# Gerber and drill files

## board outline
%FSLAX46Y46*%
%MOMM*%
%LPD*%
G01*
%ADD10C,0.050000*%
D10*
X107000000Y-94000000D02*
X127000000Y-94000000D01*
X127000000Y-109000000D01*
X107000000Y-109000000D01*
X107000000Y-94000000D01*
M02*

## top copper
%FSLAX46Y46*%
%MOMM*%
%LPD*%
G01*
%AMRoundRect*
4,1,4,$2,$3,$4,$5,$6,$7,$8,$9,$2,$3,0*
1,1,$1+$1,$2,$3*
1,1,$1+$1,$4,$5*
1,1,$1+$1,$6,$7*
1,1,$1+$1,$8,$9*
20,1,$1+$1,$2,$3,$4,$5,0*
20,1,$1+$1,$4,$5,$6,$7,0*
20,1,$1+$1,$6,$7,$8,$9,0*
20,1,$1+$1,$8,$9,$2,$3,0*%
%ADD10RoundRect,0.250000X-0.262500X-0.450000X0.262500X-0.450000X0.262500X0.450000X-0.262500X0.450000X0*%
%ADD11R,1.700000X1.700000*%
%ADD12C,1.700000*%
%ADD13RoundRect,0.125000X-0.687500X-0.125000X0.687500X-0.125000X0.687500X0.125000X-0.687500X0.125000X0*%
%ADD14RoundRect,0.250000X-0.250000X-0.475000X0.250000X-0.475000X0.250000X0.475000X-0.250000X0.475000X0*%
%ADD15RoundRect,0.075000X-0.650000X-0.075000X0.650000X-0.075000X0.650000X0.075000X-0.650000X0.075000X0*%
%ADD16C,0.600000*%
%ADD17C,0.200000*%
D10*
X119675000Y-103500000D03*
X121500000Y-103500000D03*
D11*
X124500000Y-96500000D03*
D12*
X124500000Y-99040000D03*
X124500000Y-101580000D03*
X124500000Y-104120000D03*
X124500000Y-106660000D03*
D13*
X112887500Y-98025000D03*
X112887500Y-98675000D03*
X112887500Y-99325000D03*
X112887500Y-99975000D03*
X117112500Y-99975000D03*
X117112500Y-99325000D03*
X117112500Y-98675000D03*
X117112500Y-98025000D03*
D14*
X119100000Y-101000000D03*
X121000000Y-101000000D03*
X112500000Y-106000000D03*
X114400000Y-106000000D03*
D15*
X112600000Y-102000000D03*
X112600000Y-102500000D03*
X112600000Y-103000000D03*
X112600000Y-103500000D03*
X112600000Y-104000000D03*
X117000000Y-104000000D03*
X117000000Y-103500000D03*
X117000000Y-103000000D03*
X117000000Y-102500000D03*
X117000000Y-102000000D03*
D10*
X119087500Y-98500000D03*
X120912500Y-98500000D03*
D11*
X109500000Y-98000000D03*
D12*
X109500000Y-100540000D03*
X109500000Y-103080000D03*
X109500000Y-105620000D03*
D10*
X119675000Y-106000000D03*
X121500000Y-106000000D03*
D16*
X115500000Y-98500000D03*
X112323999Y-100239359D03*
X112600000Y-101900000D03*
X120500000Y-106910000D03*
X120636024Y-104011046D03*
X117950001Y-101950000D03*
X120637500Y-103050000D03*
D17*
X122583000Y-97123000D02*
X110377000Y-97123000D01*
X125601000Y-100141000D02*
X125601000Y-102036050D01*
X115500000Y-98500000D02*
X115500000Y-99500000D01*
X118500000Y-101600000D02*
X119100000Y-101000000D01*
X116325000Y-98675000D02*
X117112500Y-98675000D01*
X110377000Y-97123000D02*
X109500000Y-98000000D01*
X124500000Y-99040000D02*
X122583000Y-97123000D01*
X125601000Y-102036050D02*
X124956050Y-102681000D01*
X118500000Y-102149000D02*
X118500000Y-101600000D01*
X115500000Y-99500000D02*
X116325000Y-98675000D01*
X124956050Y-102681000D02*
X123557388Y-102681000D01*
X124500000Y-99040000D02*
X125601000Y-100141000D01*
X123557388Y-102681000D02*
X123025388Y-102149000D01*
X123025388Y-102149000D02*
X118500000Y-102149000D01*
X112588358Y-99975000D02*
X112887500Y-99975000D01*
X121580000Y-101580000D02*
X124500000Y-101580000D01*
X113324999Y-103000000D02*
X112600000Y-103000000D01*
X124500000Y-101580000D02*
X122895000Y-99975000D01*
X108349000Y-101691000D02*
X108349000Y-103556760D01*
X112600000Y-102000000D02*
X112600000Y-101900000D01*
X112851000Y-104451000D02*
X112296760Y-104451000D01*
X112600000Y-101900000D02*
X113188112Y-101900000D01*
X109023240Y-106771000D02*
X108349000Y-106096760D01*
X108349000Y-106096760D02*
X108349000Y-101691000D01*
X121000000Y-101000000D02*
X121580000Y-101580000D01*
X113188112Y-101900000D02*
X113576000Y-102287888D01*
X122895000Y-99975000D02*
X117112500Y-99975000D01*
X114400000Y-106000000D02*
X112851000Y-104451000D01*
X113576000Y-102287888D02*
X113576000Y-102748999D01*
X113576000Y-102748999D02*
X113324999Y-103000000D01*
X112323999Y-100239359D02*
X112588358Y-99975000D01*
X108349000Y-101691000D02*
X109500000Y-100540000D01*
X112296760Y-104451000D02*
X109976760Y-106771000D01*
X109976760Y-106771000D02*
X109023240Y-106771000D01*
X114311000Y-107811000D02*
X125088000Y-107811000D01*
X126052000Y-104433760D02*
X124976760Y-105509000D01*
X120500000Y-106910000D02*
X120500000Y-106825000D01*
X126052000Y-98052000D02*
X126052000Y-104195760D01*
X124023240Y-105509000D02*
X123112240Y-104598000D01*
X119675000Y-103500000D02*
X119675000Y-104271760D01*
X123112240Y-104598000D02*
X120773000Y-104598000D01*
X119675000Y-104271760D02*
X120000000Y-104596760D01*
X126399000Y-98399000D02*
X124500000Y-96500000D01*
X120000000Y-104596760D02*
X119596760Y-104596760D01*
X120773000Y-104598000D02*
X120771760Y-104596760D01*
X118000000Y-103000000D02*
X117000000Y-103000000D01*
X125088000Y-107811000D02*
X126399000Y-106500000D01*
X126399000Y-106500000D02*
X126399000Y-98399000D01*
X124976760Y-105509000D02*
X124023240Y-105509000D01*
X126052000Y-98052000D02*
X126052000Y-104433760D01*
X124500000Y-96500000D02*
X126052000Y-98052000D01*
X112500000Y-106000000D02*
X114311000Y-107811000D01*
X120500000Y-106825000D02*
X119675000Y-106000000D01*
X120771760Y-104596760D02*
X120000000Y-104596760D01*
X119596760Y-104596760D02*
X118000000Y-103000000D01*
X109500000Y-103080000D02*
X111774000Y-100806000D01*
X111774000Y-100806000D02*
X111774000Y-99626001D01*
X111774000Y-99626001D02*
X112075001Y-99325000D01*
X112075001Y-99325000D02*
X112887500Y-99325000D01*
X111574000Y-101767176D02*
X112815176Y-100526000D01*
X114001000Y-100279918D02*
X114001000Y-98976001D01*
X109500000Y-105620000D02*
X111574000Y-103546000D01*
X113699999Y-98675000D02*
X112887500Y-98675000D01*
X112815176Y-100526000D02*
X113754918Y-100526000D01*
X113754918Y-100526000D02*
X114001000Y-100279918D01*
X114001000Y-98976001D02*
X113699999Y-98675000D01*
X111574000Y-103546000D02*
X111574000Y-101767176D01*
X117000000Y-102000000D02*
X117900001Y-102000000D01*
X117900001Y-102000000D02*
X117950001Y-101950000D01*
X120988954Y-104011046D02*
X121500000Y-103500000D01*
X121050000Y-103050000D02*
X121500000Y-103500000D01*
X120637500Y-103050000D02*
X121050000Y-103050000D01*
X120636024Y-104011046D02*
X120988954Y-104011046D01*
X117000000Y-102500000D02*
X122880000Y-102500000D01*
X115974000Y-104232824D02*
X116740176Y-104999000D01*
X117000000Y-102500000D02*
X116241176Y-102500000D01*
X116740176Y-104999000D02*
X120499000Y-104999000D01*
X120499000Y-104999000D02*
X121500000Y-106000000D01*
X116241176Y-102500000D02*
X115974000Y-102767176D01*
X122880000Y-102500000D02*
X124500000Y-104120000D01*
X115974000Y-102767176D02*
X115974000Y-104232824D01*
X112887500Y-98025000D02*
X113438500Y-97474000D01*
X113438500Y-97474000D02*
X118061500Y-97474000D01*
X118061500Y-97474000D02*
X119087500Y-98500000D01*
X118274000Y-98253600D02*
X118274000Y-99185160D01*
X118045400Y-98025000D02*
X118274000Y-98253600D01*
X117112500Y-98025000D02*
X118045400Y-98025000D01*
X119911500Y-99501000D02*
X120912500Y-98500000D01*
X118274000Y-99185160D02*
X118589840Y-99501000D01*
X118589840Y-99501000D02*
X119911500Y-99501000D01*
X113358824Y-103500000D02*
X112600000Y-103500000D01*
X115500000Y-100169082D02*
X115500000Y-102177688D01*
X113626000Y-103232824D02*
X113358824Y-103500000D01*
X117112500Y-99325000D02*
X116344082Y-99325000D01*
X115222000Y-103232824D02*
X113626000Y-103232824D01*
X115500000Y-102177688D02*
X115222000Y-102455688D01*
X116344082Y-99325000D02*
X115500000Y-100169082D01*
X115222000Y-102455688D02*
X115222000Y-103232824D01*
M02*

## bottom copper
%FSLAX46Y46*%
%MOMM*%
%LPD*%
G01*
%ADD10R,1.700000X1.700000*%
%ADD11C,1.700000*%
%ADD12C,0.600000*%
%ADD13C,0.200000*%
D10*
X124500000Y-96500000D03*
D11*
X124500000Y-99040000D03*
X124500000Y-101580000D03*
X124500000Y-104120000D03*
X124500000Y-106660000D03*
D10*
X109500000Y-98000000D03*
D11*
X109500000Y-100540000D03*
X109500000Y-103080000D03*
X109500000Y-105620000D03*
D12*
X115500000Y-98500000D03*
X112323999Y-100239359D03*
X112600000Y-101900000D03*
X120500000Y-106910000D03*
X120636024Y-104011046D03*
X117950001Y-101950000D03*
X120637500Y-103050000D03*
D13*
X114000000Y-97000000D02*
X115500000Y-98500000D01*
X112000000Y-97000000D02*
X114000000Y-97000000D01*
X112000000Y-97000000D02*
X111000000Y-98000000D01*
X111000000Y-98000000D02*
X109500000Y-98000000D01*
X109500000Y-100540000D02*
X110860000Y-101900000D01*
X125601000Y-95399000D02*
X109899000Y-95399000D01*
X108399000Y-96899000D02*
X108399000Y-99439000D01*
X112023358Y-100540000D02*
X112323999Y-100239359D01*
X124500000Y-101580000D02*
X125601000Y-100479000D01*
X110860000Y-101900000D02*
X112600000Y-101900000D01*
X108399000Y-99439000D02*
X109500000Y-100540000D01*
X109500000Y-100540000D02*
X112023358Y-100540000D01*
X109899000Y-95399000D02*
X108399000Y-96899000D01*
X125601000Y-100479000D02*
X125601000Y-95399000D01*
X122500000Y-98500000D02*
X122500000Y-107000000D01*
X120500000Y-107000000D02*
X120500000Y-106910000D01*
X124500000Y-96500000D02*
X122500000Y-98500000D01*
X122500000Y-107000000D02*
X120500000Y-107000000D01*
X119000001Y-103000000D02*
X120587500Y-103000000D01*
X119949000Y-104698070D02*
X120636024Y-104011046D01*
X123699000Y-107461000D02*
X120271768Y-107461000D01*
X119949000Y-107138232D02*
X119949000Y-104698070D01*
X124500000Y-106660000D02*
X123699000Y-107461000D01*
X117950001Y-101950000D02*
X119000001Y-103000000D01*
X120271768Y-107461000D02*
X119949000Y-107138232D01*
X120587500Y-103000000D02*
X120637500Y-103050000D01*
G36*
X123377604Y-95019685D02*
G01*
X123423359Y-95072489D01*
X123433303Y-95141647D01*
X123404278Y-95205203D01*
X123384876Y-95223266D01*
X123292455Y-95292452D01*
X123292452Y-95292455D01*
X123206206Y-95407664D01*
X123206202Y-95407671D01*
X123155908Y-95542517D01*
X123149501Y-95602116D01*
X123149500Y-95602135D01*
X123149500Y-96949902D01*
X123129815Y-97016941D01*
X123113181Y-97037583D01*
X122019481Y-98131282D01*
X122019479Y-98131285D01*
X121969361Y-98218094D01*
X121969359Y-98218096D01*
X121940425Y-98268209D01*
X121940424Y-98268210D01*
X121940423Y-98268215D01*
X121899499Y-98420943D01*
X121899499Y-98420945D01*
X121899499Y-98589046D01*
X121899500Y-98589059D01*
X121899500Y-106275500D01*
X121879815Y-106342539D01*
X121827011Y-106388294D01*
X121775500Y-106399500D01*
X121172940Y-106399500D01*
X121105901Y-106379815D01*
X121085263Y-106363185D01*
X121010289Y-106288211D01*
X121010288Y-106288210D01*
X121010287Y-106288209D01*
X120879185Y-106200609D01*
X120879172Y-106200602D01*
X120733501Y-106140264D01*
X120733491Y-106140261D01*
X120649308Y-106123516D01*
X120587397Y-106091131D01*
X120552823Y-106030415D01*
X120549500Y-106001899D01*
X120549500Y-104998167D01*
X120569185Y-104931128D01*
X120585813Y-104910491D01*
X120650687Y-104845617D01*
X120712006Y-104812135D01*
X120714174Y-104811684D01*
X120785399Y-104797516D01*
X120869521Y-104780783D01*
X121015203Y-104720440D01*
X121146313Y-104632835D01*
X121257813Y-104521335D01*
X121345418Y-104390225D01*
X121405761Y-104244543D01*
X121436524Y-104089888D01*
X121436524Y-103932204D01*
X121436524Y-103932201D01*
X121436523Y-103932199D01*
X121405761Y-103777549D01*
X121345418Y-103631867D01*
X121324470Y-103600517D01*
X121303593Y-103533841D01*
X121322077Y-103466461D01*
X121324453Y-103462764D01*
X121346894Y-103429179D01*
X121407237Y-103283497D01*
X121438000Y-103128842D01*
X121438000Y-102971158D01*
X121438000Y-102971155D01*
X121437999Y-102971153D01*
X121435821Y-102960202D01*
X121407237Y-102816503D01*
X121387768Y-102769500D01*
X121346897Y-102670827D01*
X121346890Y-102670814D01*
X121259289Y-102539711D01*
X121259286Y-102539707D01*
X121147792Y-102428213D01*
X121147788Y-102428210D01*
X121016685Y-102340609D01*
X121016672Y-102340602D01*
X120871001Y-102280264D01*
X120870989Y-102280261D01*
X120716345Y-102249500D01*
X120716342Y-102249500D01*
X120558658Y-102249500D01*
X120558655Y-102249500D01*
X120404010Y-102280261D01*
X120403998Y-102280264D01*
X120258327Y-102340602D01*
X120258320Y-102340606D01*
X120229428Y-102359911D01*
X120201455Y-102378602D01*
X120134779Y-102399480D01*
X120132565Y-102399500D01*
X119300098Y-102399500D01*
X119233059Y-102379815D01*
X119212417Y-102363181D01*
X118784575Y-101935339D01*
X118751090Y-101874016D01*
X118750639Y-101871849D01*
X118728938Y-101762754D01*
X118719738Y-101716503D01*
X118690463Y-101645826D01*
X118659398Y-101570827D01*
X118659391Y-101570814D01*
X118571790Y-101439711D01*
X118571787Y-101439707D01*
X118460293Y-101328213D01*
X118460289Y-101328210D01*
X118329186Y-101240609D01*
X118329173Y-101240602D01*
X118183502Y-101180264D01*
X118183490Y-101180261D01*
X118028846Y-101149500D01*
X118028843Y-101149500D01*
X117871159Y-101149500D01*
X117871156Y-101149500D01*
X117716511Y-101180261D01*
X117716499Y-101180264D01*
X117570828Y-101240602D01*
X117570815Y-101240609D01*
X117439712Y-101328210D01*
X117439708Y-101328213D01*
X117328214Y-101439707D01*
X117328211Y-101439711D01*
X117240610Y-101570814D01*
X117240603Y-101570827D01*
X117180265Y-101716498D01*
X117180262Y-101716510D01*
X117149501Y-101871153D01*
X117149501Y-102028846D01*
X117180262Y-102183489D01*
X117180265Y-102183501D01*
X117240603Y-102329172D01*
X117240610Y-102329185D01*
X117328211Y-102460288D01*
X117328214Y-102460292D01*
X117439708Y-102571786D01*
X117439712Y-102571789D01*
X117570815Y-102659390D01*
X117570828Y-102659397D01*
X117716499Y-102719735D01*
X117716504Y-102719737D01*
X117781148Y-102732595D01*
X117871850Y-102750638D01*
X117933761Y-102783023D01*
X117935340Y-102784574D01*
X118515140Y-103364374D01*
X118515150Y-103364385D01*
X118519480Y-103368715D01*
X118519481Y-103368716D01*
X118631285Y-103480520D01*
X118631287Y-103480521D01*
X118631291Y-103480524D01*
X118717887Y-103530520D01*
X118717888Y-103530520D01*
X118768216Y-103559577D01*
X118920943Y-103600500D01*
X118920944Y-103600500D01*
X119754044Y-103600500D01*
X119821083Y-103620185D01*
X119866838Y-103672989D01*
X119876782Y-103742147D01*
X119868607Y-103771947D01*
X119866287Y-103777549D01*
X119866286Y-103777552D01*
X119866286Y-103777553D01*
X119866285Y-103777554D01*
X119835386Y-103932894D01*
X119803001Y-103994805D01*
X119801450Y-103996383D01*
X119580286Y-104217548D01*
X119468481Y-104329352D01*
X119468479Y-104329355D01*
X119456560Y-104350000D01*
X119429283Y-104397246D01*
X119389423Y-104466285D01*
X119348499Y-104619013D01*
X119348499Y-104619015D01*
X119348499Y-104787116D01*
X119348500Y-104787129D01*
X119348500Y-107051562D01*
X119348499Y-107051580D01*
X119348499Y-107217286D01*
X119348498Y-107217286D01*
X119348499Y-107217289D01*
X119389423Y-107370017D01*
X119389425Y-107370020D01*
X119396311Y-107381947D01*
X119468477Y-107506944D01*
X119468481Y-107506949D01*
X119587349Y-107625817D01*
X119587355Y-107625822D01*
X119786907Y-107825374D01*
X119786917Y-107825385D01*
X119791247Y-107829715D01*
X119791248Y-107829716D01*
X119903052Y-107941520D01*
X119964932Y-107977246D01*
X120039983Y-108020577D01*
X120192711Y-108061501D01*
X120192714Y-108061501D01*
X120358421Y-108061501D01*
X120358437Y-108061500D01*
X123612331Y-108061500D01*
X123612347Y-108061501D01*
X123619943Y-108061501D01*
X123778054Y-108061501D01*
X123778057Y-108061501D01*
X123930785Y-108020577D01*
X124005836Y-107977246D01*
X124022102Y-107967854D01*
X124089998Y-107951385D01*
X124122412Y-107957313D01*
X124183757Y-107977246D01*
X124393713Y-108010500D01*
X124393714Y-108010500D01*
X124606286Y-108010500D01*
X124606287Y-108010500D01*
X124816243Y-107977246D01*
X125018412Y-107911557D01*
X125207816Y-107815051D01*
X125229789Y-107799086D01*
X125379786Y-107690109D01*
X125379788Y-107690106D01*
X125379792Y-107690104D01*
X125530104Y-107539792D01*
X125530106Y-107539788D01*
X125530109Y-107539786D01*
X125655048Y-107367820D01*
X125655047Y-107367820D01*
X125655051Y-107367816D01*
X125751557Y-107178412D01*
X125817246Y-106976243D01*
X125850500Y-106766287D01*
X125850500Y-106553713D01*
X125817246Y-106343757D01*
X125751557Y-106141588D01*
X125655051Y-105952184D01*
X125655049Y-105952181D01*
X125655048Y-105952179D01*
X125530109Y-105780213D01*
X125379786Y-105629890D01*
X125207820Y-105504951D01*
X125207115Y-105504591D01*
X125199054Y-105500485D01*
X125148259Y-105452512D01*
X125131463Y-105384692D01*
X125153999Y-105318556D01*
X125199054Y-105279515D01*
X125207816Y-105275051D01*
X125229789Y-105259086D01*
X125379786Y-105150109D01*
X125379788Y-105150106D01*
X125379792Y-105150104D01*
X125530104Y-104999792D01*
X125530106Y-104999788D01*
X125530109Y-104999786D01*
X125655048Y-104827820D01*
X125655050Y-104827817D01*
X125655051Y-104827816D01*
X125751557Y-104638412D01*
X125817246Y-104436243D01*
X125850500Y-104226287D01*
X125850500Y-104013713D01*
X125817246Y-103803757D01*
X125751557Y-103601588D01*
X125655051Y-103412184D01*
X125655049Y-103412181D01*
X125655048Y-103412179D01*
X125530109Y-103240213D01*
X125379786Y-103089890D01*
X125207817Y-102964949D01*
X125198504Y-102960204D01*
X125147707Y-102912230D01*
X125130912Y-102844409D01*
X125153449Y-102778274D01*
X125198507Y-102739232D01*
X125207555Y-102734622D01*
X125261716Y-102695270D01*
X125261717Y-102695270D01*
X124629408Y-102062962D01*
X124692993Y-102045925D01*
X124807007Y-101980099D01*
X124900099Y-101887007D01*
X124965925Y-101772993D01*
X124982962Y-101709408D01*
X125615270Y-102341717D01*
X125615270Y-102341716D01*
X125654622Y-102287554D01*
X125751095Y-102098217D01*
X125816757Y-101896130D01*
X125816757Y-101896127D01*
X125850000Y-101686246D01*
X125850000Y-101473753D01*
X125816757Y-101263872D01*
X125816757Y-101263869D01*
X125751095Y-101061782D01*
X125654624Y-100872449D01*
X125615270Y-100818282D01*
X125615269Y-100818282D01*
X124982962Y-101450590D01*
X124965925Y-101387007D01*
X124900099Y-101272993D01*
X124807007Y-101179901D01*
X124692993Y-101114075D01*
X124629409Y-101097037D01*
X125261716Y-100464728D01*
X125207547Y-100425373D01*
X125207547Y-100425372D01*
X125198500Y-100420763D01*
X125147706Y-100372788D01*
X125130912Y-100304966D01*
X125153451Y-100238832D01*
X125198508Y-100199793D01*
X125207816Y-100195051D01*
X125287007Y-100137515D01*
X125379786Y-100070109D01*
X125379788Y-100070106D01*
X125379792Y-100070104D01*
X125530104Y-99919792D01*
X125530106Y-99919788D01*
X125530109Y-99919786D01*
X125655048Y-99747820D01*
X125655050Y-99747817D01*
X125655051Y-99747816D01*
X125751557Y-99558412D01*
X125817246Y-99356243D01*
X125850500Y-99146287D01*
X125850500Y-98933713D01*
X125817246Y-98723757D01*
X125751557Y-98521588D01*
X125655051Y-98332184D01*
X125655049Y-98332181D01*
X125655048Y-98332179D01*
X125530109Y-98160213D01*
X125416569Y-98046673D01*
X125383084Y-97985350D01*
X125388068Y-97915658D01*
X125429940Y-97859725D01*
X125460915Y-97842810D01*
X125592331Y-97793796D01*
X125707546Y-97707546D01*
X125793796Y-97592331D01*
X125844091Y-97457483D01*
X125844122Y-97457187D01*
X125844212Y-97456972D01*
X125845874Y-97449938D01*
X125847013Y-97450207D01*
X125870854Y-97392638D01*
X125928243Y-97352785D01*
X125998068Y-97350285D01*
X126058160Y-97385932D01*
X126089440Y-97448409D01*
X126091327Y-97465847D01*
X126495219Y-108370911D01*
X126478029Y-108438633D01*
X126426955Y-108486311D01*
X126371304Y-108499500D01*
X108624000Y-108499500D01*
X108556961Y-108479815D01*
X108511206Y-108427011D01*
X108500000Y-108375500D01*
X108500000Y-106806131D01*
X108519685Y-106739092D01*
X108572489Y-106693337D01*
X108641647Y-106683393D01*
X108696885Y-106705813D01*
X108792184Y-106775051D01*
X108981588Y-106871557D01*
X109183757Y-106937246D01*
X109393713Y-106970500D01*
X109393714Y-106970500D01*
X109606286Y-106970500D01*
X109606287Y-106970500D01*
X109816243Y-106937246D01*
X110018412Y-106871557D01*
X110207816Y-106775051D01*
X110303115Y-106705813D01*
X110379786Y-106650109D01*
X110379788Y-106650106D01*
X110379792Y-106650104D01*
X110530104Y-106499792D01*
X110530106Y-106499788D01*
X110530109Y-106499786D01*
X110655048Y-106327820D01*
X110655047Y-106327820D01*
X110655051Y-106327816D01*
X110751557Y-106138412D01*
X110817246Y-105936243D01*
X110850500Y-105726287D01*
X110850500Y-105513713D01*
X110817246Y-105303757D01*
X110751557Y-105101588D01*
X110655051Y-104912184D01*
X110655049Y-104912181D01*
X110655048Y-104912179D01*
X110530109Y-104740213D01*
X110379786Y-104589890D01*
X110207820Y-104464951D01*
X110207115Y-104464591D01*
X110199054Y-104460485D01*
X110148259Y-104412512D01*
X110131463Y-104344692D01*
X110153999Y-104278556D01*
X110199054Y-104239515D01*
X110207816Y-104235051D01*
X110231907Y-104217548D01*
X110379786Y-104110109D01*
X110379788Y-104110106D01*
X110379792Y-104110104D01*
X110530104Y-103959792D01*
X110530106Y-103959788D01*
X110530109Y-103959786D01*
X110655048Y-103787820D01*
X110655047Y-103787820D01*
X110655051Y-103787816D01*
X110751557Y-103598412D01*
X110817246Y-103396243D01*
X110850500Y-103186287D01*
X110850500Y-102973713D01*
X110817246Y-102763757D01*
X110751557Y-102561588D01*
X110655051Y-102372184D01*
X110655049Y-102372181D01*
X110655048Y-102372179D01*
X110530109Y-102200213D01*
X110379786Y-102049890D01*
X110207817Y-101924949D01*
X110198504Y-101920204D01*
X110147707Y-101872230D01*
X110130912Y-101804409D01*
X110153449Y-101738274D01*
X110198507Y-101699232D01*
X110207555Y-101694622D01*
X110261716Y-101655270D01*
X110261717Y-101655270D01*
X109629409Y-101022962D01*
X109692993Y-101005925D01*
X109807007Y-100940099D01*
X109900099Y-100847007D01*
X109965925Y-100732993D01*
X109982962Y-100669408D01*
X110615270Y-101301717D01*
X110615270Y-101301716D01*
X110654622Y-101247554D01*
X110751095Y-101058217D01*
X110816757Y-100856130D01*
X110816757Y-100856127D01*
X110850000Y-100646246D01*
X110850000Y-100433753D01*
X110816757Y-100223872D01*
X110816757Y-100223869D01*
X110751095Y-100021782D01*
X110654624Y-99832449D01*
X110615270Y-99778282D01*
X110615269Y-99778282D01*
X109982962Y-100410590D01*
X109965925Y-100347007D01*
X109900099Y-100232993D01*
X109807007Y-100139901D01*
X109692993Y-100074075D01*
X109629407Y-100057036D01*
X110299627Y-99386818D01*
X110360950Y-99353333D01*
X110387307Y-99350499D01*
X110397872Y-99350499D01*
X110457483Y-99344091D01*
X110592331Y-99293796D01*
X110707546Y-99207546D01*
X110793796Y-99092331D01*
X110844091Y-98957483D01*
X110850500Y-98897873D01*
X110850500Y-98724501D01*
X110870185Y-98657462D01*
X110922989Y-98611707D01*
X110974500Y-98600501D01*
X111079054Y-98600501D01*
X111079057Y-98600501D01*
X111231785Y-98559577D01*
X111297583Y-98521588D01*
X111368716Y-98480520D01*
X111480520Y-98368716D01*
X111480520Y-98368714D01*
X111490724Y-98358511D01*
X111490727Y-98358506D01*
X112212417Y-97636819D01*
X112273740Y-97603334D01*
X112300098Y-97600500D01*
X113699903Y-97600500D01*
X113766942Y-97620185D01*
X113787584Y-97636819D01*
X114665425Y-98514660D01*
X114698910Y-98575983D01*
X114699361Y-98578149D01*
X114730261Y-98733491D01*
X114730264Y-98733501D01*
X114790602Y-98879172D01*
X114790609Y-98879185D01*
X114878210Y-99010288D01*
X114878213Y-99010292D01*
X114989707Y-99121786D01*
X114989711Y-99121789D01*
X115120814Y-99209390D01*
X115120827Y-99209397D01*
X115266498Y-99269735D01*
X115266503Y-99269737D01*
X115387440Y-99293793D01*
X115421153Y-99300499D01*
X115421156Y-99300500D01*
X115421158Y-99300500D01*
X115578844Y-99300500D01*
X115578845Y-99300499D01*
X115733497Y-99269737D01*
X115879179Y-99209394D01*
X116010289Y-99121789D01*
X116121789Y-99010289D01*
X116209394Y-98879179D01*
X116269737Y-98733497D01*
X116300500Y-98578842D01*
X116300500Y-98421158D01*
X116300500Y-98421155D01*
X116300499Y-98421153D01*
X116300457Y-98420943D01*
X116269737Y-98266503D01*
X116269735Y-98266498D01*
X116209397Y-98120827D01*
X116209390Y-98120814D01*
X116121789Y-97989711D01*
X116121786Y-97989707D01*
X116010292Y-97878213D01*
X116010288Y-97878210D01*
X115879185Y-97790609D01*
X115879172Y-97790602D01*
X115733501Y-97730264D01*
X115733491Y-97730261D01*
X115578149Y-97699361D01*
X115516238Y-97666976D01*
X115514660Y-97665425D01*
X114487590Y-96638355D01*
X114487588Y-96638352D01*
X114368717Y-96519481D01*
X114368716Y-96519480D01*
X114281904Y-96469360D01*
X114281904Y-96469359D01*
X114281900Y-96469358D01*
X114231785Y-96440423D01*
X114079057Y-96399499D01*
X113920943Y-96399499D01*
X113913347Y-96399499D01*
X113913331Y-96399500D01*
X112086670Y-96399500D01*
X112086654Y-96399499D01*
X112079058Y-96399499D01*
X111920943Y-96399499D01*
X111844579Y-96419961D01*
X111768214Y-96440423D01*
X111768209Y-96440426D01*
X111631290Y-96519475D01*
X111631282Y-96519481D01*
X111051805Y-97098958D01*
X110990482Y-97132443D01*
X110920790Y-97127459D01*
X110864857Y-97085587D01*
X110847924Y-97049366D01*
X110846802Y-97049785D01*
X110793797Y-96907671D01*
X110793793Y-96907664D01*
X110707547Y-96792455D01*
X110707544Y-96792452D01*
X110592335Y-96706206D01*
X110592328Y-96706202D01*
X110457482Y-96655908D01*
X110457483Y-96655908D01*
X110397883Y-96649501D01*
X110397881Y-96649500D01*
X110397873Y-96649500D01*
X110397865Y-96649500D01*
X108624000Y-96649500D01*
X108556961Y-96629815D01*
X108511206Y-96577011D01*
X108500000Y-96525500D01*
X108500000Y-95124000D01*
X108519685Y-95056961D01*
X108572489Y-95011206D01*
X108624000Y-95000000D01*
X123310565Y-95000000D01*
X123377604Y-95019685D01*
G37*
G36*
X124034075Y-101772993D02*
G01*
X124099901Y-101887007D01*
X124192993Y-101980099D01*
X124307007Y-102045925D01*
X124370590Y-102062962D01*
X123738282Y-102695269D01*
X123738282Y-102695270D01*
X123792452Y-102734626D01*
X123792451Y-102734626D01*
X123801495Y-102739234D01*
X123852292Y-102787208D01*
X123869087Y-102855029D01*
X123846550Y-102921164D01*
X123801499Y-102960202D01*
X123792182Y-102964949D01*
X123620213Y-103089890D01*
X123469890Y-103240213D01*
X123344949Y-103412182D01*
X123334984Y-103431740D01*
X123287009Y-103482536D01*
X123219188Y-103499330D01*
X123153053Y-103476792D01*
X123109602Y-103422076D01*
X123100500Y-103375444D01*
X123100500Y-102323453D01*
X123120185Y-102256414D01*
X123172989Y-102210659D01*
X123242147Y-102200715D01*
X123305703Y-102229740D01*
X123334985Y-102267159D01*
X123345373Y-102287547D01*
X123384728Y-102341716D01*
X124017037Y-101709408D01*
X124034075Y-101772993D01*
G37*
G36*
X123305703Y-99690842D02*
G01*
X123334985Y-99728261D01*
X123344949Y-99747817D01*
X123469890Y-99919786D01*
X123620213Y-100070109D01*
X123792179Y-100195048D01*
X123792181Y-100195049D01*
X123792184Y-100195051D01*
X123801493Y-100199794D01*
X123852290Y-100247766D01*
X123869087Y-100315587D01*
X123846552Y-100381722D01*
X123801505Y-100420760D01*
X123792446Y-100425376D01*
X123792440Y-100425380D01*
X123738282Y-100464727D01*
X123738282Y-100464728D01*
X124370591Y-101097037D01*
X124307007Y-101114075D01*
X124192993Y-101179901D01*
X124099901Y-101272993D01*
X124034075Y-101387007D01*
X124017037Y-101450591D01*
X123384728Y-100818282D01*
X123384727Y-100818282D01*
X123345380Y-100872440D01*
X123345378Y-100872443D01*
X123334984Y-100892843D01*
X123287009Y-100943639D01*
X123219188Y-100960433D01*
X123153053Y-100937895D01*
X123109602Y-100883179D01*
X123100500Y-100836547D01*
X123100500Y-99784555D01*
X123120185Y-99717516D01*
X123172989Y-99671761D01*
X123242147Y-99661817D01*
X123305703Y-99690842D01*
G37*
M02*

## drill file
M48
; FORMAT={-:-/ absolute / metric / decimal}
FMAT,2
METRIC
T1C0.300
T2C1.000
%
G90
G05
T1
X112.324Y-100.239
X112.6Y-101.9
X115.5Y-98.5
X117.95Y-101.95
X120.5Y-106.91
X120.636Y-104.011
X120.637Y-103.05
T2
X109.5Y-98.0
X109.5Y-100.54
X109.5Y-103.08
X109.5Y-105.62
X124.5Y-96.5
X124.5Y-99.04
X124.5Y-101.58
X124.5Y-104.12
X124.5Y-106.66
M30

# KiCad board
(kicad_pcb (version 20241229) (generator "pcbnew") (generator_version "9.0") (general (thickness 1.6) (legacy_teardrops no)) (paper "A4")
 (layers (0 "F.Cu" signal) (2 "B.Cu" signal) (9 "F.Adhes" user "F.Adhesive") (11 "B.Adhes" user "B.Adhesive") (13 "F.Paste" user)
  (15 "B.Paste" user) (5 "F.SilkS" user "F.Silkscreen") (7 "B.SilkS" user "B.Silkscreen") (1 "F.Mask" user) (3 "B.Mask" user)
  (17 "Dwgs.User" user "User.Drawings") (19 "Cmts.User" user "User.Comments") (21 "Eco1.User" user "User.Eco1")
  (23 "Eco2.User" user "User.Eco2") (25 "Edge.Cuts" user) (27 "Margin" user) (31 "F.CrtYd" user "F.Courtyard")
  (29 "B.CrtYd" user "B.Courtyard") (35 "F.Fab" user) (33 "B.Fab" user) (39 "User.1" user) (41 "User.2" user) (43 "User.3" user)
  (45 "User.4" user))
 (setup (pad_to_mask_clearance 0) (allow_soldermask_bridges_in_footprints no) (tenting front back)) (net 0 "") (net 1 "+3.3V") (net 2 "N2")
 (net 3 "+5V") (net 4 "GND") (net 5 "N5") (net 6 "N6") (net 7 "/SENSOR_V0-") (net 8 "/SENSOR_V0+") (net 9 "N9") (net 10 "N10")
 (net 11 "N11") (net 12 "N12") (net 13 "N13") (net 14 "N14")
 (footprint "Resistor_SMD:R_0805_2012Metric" (layer "F.Cu") (at 120.5875 103.5)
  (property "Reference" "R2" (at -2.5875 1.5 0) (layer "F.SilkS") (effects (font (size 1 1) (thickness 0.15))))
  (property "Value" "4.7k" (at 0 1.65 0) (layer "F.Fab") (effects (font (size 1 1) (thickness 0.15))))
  (pad "1" smd roundrect (at -0.9125 0) (size 1.025 1.4) (layers "F.Cu" "F.Mask" "F.Paste") (roundrect_rratio 0.243902) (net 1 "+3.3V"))
  (pad "2" smd roundrect (at 0.9125 0) (size 1.025 1.4) (layers "F.Cu" "F.Mask" "F.Paste") (roundrect_rratio 0.243902) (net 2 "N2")))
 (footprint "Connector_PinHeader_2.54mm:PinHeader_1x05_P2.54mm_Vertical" (layer "F.Cu") (at 124.5 96.5)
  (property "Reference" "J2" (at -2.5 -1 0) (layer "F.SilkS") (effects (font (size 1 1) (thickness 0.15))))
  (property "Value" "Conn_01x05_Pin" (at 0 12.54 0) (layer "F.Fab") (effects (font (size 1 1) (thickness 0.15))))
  (pad "1" thru_hole rect (at 0 0) (size 1.7 1.7) (drill 1) (layers "*.Cu" "*.Mask") (remove_unused_layers no) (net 1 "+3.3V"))
  (pad "2" thru_hole circle (at 0 2.54) (size 1.7 1.7) (drill 1) (layers "*.Cu" "*.Mask") (remove_unused_layers no) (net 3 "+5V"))
  (pad "3" thru_hole circle (at 0 5.08) (size 1.7 1.7) (drill 1) (layers "*.Cu" "*.Mask") (remove_unused_layers no) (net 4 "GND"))
  (pad "4" thru_hole circle (at 0 7.62) (size 1.7 1.7) (drill 1) (layers "*.Cu" "*.Mask") (remove_unused_layers no) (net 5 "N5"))
  (pad "5" thru_hole circle (at 0 10.16) (size 1.7 1.7) (drill 1) (layers "*.Cu" "*.Mask") (remove_unused_layers no) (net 2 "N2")))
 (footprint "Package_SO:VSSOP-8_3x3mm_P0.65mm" (layer "F.Cu") (at 115 99)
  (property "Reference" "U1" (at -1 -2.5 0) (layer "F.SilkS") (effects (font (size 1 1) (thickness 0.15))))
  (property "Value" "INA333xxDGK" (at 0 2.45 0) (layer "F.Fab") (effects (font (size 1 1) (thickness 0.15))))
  (pad "1" smd roundrect (at -2.1125 -0.975) (size 1.625 0.5) (layers "F.Cu" "F.Mask" "F.Paste") (roundrect_rratio 0.25) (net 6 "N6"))
  (pad "2" smd roundrect (at -2.1125 -0.325) (size 1.625 0.5) (layers "F.Cu" "F.Mask" "F.Paste") (roundrect_rratio 0.25)
   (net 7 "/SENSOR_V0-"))
  (pad "3" smd roundrect (at -2.1125 0.325) (size 1.625 0.5) (layers "F.Cu" "F.Mask" "F.Paste") (roundrect_rratio 0.25)
   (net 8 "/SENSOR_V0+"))
  (pad "4" smd roundrect (at -2.1125 0.975) (size 1.625 0.5) (layers "F.Cu" "F.Mask" "F.Paste") (roundrect_rratio 0.25) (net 4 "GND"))
  (pad "5" smd roundrect (at 2.1125 0.975) (size 1.625 0.5) (layers "F.Cu" "F.Mask" "F.Paste") (roundrect_rratio 0.25) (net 4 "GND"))
  (pad "6" smd roundrect (at 2.1125 0.325) (size 1.625 0.5) (layers "F.Cu" "F.Mask" "F.Paste") (roundrect_rratio 0.25) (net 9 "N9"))
  (pad "7" smd roundrect (at 2.1125 -0.325) (size 1.625 0.5) (layers "F.Cu" "F.Mask" "F.Paste") (roundrect_rratio 0.25) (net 3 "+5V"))
  (pad "8" smd roundrect (at 2.1125 -0.975) (size 1.625 0.5) (layers "F.Cu" "F.Mask" "F.Paste") (roundrect_rratio 0.25) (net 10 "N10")))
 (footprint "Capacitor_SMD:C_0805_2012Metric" (layer "F.Cu") (at 120.05 101)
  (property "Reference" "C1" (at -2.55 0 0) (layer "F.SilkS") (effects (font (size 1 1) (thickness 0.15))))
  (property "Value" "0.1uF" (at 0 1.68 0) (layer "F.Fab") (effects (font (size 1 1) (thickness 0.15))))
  (pad "1" smd roundrect (at -0.95 0) (size 1 1.45) (layers "F.Cu" "F.Mask" "F.Paste") (roundrect_rratio 0.25) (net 3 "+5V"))
  (pad "2" smd roundrect (at 0.95 0) (size 1 1.45) (layers "F.Cu" "F.Mask" "F.Paste") (roundrect_rratio 0.25) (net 4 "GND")))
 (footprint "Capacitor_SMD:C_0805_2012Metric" (layer "F.Cu") (at 113.45 106)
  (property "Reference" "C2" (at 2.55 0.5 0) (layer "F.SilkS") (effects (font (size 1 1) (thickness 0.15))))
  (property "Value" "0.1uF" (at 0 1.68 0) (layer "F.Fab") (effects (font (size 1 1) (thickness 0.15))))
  (pad "1" smd roundrect (at -0.95 0) (size 1 1.45) (layers "F.Cu" "F.Mask" "F.Paste") (roundrect_rratio 0.25) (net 1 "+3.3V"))
  (pad "2" smd roundrect (at 0.95 0) (size 1 1.45) (layers "F.Cu" "F.Mask" "F.Paste") (roundrect_rratio 0.25) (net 4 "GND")))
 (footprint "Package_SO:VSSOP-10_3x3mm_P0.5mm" (layer "F.Cu") (at 114.8 103)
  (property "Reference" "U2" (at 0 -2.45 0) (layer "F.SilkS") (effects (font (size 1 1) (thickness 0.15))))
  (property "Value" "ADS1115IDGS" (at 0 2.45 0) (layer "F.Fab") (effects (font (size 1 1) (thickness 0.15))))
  (pad "1" smd roundrect (at -2.2 -1) (size 1.45 0.3) (layers "F.Cu" "F.Mask" "F.Paste") (roundrect_rratio 0.25) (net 4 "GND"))
  (pad "2" smd roundrect (at -2.2 -0.5) (size 1.45 0.3) (layers "F.Cu" "F.Mask" "F.Paste") (roundrect_rratio 0.25) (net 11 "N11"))
  (pad "3" smd roundrect (at -2.2 0) (size 1.45 0.3) (layers "F.Cu" "F.Mask" "F.Paste") (roundrect_rratio 0.25) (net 4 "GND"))
  (pad "4" smd roundrect (at -2.2 0.5) (size 1.45 0.3) (layers "F.Cu" "F.Mask" "F.Paste") (roundrect_rratio 0.25) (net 9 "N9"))
  (pad "5" smd roundrect (at -2.2 1) (size 1.45 0.3) (layers "F.Cu" "F.Mask" "F.Paste") (roundrect_rratio 0.25) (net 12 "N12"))
  (pad "6" smd roundrect (at 2.2 1) (size 1.45 0.3) (layers "F.Cu" "F.Mask" "F.Paste") (roundrect_rratio 0.25) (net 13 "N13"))
  (pad "7" smd roundrect (at 2.2 0.5) (size 1.45 0.3) (layers "F.Cu" "F.Mask" "F.Paste") (roundrect_rratio 0.25) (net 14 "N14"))
  (pad "8" smd roundrect (at 2.2 0) (size 1.45 0.3) (layers "F.Cu" "F.Mask" "F.Paste") (roundrect_rratio 0.25) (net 1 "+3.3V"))
  (pad "9" smd roundrect (at 2.2 -0.5) (size 1.45 0.3) (layers "F.Cu" "F.Mask" "F.Paste") (roundrect_rratio 0.25) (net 5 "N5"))
  (pad "10" smd roundrect (at 2.2 -1) (size 1.45 0.3) (layers "F.Cu" "F.Mask" "F.Paste") (roundrect_rratio 0.25) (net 2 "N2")))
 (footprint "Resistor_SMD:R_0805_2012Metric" (layer "F.Cu") (at 120 98.5)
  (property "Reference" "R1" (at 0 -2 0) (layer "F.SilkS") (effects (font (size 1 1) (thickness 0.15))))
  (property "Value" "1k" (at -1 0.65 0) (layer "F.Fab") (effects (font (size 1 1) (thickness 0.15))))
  (pad "1" smd roundrect (at -0.9125 0) (size 1.025 1.4) (layers "F.Cu" "F.Mask" "F.Paste") (roundrect_rratio 0.243902) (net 6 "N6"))
  (pad "2" smd roundrect (at 0.9125 0) (size 1.025 1.4) (layers "F.Cu" "F.Mask" "F.Paste") (roundrect_rratio 0.243902) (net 10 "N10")))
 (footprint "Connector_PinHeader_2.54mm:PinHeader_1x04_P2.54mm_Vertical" (layer "F.Cu") (at 109.5 98)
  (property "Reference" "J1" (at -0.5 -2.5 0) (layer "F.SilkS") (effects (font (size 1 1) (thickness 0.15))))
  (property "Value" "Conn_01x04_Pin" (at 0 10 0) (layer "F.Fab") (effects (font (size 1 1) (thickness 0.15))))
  (pad "1" thru_hole rect (at 0 0) (size 1.7 1.7) (drill 1) (layers "*.Cu" "*.Mask") (remove_unused_layers no) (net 3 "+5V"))
  (pad "2" thru_hole circle (at 0 2.54) (size 1.7 1.7) (drill 1) (layers "*.Cu" "*.Mask") (remove_unused_layers no) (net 4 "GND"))
  (pad "3" thru_hole circle (at 0 5.08) (size 1.7 1.7) (drill 1) (layers "*.Cu" "*.Mask") (remove_unused_layers no) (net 8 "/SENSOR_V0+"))
  (pad "4" thru_hole circle (at 0 7.62) (size 1.7 1.7) (drill 1) (layers "*.Cu" "*.Mask") (remove_unused_layers no) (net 7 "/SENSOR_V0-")))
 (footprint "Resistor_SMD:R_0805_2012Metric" (layer "F.Cu") (at 120.5875 106)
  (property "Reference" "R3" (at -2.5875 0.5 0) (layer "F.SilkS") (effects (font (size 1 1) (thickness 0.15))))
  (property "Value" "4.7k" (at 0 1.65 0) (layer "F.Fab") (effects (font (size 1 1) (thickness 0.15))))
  (pad "1" smd roundrect (at -0.9125 0) (size 1.025 1.4) (layers "F.Cu" "F.Mask" "F.Paste") (roundrect_rratio 0.243902) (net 1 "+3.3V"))
  (pad "2" smd roundrect (at 0.9125 0) (size 1.025 1.4) (layers "F.Cu" "F.Mask" "F.Paste") (roundrect_rratio 0.243902) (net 5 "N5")))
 (gr_rect (start 107 94) (end 127 109) (stroke (width 0.05) (type default)) (fill no) (layer "Edge.Cuts"))
 (segment (start 122.583 97.123) (end 110.377 97.123) (width 0.2) (layer "F.Cu") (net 3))
 (segment (start 125.601 100.141) (end 125.601 102.03605) (width 0.2) (layer "F.Cu") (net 3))
 (segment (start 115.5 98.5) (end 115.5 99.5) (width 0.2) (layer "F.Cu") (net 3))
 (segment (start 118.5 101.6) (end 119.1 101) (width 0.2) (layer "F.Cu") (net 3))
 (segment (start 116.325 98.675) (end 117.1125 98.675) (width 0.2) (layer "F.Cu") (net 3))
 (segment (start 110.377 97.123) (end 109.5 98) (width 0.2) (layer "F.Cu") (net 3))
 (segment (start 124.5 99.04) (end 122.583 97.123) (width 0.2) (layer "F.Cu") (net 3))
 (segment (start 125.601 102.03605) (end 124.95605 102.681) (width 0.2) (layer "F.Cu") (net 3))
 (segment (start 118.5 102.149) (end 118.5 101.6) (width 0.2) (layer "F.Cu") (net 3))
 (segment (start 115.5 99.5) (end 116.325 98.675) (width 0.2) (layer "F.Cu") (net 3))
 (segment (start 124.95605 102.681) (end 123.557388 102.681) (width 0.2) (layer "F.Cu") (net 3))
 (segment (start 124.5 99.04) (end 125.601 100.141) (width 0.2) (layer "F.Cu") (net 3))
 (segment (start 123.557388 102.681) (end 123.025388 102.149) (width 0.2) (layer "F.Cu") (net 3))
 (segment (start 123.025388 102.149) (end 118.5 102.149) (width 0.2) (layer "F.Cu") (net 3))
 (via (at 115.5 98.5) (size 0.6) (drill 0.3) (layers "F.Cu" "B.Cu") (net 3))
 (segment (start 114 97) (end 115.5 98.5) (width 0.2) (layer "B.Cu") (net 3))
 (segment (start 112 97) (end 114 97) (width 0.2) (layer "B.Cu") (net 3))
 (segment (start 112 97) (end 111 98) (width 0.2) (layer "B.Cu") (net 3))
 (segment (start 111 98) (end 109.5 98) (width 0.2) (layer "B.Cu") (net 3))
 (segment (start 112.588358 99.975) (end 112.8875 99.975) (width 0.2) (layer "F.Cu") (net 4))
 (segment (start 121.58 101.58) (end 124.5 101.58) (width 0.2) (layer "F.Cu") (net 4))
 (segment (start 113.324999 103) (end 112.6 103) (width 0.2) (layer "F.Cu") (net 4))
 (segment (start 124.5 101.58) (end 122.895 99.975) (width 0.2) (layer "F.Cu") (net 4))
 (segment (start 108.349 101.691) (end 108.349 103.55676) (width 0.2) (layer "F.Cu") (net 4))
 (segment (start 112.6 102) (end 112.6 101.9) (width 0.2) (layer "F.Cu") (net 4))
 (segment (start 112.851 104.451) (end 112.29676 104.451) (width 0.2) (layer "F.Cu") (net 4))
 (segment (start 112.6 101.9) (end 113.188112 101.9) (width 0.2) (layer "F.Cu") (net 4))
 (segment (start 109.02324 106.771) (end 108.349 106.09676) (width 0.2) (layer "F.Cu") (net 4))
 (segment (start 108.349 106.09676) (end 108.349 101.691) (width 0.2) (layer "F.Cu") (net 4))
 (segment (start 121 101) (end 121.58 101.58) (width 0.2) (layer "F.Cu") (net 4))
 (segment (start 113.188112 101.9) (end 113.576 102.287888) (width 0.2) (layer "F.Cu") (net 4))
 (segment (start 122.895 99.975) (end 117.1125 99.975) (width 0.2) (layer "F.Cu") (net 4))
 (segment (start 114.4 106) (end 112.851 104.451) (width 0.2) (layer "F.Cu") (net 4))
 (segment (start 113.576 102.287888) (end 113.576 102.748999) (width 0.2) (layer "F.Cu") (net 4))
 (segment (start 113.576 102.748999) (end 113.324999 103) (width 0.2) (layer "F.Cu") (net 4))
 (segment (start 112.323999 100.239359) (end 112.588358 99.975) (width 0.2) (layer "F.Cu") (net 4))
 (segment (start 108.349 101.691) (end 109.5 100.54) (width 0.2) (layer "F.Cu") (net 4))
 (segment (start 112.29676 104.451) (end 109.97676 106.771) (width 0.2) (layer "F.Cu") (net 4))
 (segment (start 109.97676 106.771) (end 109.02324 106.771) (width 0.2) (layer "F.Cu") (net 4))
 (via (at 112.323999 100.239359) (size 0.6) (drill 0.3) (layers "F.Cu" "B.Cu") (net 4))
 (via (at 112.6 101.9) (size 0.6) (drill 0.3) (layers "F.Cu" "B.Cu") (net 4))
 (segment (start 109.5 100.54) (end 110.86 101.9) (width 0.2) (layer "B.Cu") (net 4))
 (segment (start 125.601 95.399) (end 109.899 95.399) (width 0.2) (layer "B.Cu") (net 4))
 (segment (start 108.399 96.899) (end 108.399 99.439) (width 0.2) (layer "B.Cu") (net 4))
 (segment (start 112.023358 100.54) (end 112.323999 100.239359) (width 0.2) (layer "B.Cu") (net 4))
 (segment (start 124.5 101.58) (end 125.601 100.479) (width 0.2) (layer "B.Cu") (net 4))
 (segment (start 110.86 101.9) (end 112.6 101.9) (width 0.2) (layer "B.Cu") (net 4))
 (segment (start 108.399 99.439) (end 109.5 100.54) (width 0.2) (layer "B.Cu") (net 4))
 (segment (start 109.5 100.54) (end 112.023358 100.54) (width 0.2) (layer "B.Cu") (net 4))
 (segment (start 109.899 95.399) (end 108.399 96.899) (width 0.2) (layer "B.Cu") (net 4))
 (segment (start 125.601 100.479) (end 125.601 95.399) (width 0.2) (layer "B.Cu") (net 4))
 (segment (start 114.311 107.811) (end 125.088 107.811) (width 0.2) (layer "F.Cu") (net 1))
 (segment (start 126.052 104.43376) (end 124.97676 105.509) (width 0.2) (layer "F.Cu") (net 1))
 (segment (start 120.5 106.91) (end 120.5 106.825) (width 0.2) (layer "F.Cu") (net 1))
 (segment (start 126.052 98.052) (end 126.052 104.19576) (width 0.2) (layer "F.Cu") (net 1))
 (segment (start 124.02324 105.509) (end 123.11224 104.598) (width 0.2) (layer "F.Cu") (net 1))
 (segment (start 119.675 103.5) (end 119.675 104.27176) (width 0.2) (layer "F.Cu") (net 1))
 (segment (start 123.11224 104.598) (end 120.773 104.598) (width 0.2) (layer "F.Cu") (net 1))
 (segment (start 119.675 104.27176) (end 120 104.59676) (width 0.2) (layer "F.Cu") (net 1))
 (segment (start 126.399 98.399) (end 124.5 96.5) (width 0.2) (layer "F.Cu") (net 1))
 (segment (start 120 104.59676) (end 119.59676 104.59676) (width 0.2) (layer "F.Cu") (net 1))
 (segment (start 120.773 104.598) (end 120.77176 104.59676) (width 0.2) (layer "F.Cu") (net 1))
 (segment (start 118 103) (end 117 103) (width 0.2) (layer "F.Cu") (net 1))
 (segment (start 125.088 107.811) (end 126.399 106.5) (width 0.2) (layer "F.Cu") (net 1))
 (segment (start 126.399 106.5) (end 126.399 98.399) (width 0.2) (layer "F.Cu") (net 1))
 (segment (start 124.97676 105.509) (end 124.02324 105.509) (width 0.2) (layer "F.Cu") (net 1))
 (segment (start 126.052 98.052) (end 126.052 104.43376) (width 0.2) (layer "F.Cu") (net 1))
 (segment (start 124.5 96.5) (end 126.052 98.052) (width 0.2) (layer "F.Cu") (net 1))
 (segment (start 112.5 106) (end 114.311 107.811) (width 0.2) (layer "F.Cu") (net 1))
 (segment (start 120.5 106.825) (end 119.675 106) (width 0.2) (layer "F.Cu") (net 1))
 (segment (start 120.77176 104.59676) (end 120 104.59676) (width 0.2) (layer "F.Cu") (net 1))
 (segment (start 119.59676 104.59676) (end 118 103) (width 0.2) (layer "F.Cu") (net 1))
 (via (at 120.5 106.91) (size 0.6) (drill 0.3) (layers "F.Cu" "B.Cu") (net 1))
 (segment (start 122.5 98.5) (end 122.5 107) (width 0.2) (layer "B.Cu") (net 1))
 (segment (start 120.5 107) (end 120.5 106.91) (width 0.2) (layer "B.Cu") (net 1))
 (segment (start 124.5 96.5) (end 122.5 98.5) (width 0.2) (layer "B.Cu") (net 1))
 (segment (start 122.5 107) (end 120.5 107) (width 0.2) (layer "B.Cu") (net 1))
 (segment (start 109.5 103.08) (end 111.774 100.806) (width 0.2) (layer "F.Cu") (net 8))
 (segment (start 111.774 100.806) (end 111.774 99.626001) (width 0.2) (layer "F.Cu") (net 8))
 (segment (start 111.774 99.626001) (end 112.075001 99.325) (width 0.2) (layer "F.Cu") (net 8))
 (segment (start 112.075001 99.325) (end 112.8875 99.325) (width 0.2) (layer "F.Cu") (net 8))
 (segment (start 111.574 101.767176) (end 112.815176 100.526) (width 0.2) (layer "F.Cu") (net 7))
 (segment (start 114.001 100.279918) (end 114.001 98.976001) (width 0.2) (layer "F.Cu") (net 7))
 (segment (start 109.5 105.62) (end 111.574 103.546) (width 0.2) (layer "F.Cu") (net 7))
 (segment (start 113.699999 98.675) (end 112.8875 98.675) (width 0.2) (layer "F.Cu") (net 7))
 (segment (start 112.815176 100.526) (end 113.754918 100.526) (width 0.2) (layer "F.Cu") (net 7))
 (segment (start 113.754918 100.526) (end 114.001 100.279918) (width 0.2) (layer "F.Cu") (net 7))
 (segment (start 114.001 98.976001) (end 113.699999 98.675) (width 0.2) (layer "F.Cu") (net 7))
 (segment (start 111.574 103.546) (end 111.574 101.767176) (width 0.2) (layer "F.Cu") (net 7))
 (segment (start 117 102) (end 117.900001 102) (width 0.2) (layer "F.Cu") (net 2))
 (segment (start 117.900001 102) (end 117.950001 101.95) (width 0.2) (layer "F.Cu") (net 2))
 (segment (start 120.988954 104.011046) (end 121.5 103.5) (width 0.2) (layer "F.Cu") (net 2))
 (segment (start 121.05 103.05) (end 121.5 103.5) (width 0.2) (layer "F.Cu") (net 2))
 (segment (start 120.6375 103.05) (end 121.05 103.05) (width 0.2) (layer "F.Cu") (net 2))
 (segment (start 120.636024 104.011046) (end 120.988954 104.011046) (width 0.2) (layer "F.Cu") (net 2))
 (via (at 120.636024 104.011046) (size 0.6) (drill 0.3) (layers "F.Cu" "B.Cu") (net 2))
 (via (at 117.950001 101.95) (size 0.6) (drill 0.3) (layers "F.Cu" "B.Cu") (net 2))
 (via (at 120.6375 103.05) (size 0.6) (drill 0.3) (layers "F.Cu" "B.Cu") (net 2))
 (segment (start 119.000001 103) (end 120.5875 103) (width 0.2) (layer "B.Cu") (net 2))
 (segment (start 119.949 104.69807) (end 120.636024 104.011046) (width 0.2) (layer "B.Cu") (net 2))
 (segment (start 123.699 107.461) (end 120.271768 107.461) (width 0.2) (layer "B.Cu") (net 2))
 (segment (start 119.949 107.138232) (end 119.949 104.69807) (width 0.2) (layer "B.Cu") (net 2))
 (segment (start 124.5 106.66) (end 123.699 107.461) (width 0.2) (layer "B.Cu") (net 2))
 (segment (start 117.950001 101.95) (end 119.000001 103) (width 0.2) (layer "B.Cu") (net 2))
 (segment (start 120.271768 107.461) (end 119.949 107.138232) (width 0.2) (layer "B.Cu") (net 2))
 (segment (start 120.5875 103) (end 120.6375 103.05) (width 0.2) (layer "B.Cu") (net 2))
 (segment (start 117 102.5) (end 122.88 102.5) (width 0.2) (layer "F.Cu") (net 5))
 (segment (start 115.974 104.232824) (end 116.740176 104.999) (width 0.2) (layer "F.Cu") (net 5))
 (segment (start 117 102.5) (end 116.241176 102.5) (width 0.2) (layer "F.Cu") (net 5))
 (segment (start 116.740176 104.999) (end 120.499 104.999) (width 0.2) (layer "F.Cu") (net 5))
 (segment (start 120.499 104.999) (end 121.5 106) (width 0.2) (layer "F.Cu") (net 5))
 (segment (start 116.241176 102.5) (end 115.974 102.767176) (width 0.2) (layer "F.Cu") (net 5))
 (segment (start 122.88 102.5) (end 124.5 104.12) (width 0.2) (layer "F.Cu") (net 5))
 (segment (start 115.974 102.767176) (end 115.974 104.232824) (width 0.2) (layer "F.Cu") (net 5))
 (segment (start 112.8875 98.025) (end 113.4385 97.474) (width 0.2) (layer "F.Cu") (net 6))
 (segment (start 113.4385 97.474) (end 118.0615 97.474) (width 0.2) (layer "F.Cu") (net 6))
 (segment (start 118.0615 97.474) (end 119.0875 98.5) (width 0.2) (layer "F.Cu") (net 6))
 (segment (start 118.274 98.2536) (end 118.274 99.18516) (width 0.2) (layer "F.Cu") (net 10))
 (segment (start 118.0454 98.025) (end 118.274 98.2536) (width 0.2) (layer "F.Cu") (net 10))
 (segment (start 117.1125 98.025) (end 118.0454 98.025) (width 0.2) (layer "F.Cu") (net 10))
 (segment (start 119.9115 99.501) (end 120.9125 98.5) (width 0.2) (layer "F.Cu") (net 10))
 (segment (start 118.274 99.18516) (end 118.58984 99.501) (width 0.2) (layer "F.Cu") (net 10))
 (segment (start 118.58984 99.501) (end 119.9115 99.501) (width 0.2) (layer "F.Cu") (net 10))
 (segment (start 113.358824 103.5) (end 112.6 103.5) (width 0.2) (layer "F.Cu") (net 9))
 (segment (start 115.5 100.169082) (end 115.5 102.177688) (width 0.2) (layer "F.Cu") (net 9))
 (segment (start 113.626 103.232824) (end 113.358824 103.5) (width 0.2) (layer "F.Cu") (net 9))
 (segment (start 117.1125 99.325) (end 116.344082 99.325) (width 0.2) (layer "F.Cu") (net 9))
 (segment (start 115.222 103.232824) (end 113.626 103.232824) (width 0.2) (layer "F.Cu") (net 9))
 (segment (start 115.5 102.177688) (end 115.222 102.455688) (width 0.2) (layer "F.Cu") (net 9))
 (segment (start 116.344082 99.325) (end 115.5 100.169082) (width 0.2) (layer "F.Cu") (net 9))
 (segment (start 115.222 102.455688) (end 115.222 103.232824) (width 0.2) (layer "F.Cu") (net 9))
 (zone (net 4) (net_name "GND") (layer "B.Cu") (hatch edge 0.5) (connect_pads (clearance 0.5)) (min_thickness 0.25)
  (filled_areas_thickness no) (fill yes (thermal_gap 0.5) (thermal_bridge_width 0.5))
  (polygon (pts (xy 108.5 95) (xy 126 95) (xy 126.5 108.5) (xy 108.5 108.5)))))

